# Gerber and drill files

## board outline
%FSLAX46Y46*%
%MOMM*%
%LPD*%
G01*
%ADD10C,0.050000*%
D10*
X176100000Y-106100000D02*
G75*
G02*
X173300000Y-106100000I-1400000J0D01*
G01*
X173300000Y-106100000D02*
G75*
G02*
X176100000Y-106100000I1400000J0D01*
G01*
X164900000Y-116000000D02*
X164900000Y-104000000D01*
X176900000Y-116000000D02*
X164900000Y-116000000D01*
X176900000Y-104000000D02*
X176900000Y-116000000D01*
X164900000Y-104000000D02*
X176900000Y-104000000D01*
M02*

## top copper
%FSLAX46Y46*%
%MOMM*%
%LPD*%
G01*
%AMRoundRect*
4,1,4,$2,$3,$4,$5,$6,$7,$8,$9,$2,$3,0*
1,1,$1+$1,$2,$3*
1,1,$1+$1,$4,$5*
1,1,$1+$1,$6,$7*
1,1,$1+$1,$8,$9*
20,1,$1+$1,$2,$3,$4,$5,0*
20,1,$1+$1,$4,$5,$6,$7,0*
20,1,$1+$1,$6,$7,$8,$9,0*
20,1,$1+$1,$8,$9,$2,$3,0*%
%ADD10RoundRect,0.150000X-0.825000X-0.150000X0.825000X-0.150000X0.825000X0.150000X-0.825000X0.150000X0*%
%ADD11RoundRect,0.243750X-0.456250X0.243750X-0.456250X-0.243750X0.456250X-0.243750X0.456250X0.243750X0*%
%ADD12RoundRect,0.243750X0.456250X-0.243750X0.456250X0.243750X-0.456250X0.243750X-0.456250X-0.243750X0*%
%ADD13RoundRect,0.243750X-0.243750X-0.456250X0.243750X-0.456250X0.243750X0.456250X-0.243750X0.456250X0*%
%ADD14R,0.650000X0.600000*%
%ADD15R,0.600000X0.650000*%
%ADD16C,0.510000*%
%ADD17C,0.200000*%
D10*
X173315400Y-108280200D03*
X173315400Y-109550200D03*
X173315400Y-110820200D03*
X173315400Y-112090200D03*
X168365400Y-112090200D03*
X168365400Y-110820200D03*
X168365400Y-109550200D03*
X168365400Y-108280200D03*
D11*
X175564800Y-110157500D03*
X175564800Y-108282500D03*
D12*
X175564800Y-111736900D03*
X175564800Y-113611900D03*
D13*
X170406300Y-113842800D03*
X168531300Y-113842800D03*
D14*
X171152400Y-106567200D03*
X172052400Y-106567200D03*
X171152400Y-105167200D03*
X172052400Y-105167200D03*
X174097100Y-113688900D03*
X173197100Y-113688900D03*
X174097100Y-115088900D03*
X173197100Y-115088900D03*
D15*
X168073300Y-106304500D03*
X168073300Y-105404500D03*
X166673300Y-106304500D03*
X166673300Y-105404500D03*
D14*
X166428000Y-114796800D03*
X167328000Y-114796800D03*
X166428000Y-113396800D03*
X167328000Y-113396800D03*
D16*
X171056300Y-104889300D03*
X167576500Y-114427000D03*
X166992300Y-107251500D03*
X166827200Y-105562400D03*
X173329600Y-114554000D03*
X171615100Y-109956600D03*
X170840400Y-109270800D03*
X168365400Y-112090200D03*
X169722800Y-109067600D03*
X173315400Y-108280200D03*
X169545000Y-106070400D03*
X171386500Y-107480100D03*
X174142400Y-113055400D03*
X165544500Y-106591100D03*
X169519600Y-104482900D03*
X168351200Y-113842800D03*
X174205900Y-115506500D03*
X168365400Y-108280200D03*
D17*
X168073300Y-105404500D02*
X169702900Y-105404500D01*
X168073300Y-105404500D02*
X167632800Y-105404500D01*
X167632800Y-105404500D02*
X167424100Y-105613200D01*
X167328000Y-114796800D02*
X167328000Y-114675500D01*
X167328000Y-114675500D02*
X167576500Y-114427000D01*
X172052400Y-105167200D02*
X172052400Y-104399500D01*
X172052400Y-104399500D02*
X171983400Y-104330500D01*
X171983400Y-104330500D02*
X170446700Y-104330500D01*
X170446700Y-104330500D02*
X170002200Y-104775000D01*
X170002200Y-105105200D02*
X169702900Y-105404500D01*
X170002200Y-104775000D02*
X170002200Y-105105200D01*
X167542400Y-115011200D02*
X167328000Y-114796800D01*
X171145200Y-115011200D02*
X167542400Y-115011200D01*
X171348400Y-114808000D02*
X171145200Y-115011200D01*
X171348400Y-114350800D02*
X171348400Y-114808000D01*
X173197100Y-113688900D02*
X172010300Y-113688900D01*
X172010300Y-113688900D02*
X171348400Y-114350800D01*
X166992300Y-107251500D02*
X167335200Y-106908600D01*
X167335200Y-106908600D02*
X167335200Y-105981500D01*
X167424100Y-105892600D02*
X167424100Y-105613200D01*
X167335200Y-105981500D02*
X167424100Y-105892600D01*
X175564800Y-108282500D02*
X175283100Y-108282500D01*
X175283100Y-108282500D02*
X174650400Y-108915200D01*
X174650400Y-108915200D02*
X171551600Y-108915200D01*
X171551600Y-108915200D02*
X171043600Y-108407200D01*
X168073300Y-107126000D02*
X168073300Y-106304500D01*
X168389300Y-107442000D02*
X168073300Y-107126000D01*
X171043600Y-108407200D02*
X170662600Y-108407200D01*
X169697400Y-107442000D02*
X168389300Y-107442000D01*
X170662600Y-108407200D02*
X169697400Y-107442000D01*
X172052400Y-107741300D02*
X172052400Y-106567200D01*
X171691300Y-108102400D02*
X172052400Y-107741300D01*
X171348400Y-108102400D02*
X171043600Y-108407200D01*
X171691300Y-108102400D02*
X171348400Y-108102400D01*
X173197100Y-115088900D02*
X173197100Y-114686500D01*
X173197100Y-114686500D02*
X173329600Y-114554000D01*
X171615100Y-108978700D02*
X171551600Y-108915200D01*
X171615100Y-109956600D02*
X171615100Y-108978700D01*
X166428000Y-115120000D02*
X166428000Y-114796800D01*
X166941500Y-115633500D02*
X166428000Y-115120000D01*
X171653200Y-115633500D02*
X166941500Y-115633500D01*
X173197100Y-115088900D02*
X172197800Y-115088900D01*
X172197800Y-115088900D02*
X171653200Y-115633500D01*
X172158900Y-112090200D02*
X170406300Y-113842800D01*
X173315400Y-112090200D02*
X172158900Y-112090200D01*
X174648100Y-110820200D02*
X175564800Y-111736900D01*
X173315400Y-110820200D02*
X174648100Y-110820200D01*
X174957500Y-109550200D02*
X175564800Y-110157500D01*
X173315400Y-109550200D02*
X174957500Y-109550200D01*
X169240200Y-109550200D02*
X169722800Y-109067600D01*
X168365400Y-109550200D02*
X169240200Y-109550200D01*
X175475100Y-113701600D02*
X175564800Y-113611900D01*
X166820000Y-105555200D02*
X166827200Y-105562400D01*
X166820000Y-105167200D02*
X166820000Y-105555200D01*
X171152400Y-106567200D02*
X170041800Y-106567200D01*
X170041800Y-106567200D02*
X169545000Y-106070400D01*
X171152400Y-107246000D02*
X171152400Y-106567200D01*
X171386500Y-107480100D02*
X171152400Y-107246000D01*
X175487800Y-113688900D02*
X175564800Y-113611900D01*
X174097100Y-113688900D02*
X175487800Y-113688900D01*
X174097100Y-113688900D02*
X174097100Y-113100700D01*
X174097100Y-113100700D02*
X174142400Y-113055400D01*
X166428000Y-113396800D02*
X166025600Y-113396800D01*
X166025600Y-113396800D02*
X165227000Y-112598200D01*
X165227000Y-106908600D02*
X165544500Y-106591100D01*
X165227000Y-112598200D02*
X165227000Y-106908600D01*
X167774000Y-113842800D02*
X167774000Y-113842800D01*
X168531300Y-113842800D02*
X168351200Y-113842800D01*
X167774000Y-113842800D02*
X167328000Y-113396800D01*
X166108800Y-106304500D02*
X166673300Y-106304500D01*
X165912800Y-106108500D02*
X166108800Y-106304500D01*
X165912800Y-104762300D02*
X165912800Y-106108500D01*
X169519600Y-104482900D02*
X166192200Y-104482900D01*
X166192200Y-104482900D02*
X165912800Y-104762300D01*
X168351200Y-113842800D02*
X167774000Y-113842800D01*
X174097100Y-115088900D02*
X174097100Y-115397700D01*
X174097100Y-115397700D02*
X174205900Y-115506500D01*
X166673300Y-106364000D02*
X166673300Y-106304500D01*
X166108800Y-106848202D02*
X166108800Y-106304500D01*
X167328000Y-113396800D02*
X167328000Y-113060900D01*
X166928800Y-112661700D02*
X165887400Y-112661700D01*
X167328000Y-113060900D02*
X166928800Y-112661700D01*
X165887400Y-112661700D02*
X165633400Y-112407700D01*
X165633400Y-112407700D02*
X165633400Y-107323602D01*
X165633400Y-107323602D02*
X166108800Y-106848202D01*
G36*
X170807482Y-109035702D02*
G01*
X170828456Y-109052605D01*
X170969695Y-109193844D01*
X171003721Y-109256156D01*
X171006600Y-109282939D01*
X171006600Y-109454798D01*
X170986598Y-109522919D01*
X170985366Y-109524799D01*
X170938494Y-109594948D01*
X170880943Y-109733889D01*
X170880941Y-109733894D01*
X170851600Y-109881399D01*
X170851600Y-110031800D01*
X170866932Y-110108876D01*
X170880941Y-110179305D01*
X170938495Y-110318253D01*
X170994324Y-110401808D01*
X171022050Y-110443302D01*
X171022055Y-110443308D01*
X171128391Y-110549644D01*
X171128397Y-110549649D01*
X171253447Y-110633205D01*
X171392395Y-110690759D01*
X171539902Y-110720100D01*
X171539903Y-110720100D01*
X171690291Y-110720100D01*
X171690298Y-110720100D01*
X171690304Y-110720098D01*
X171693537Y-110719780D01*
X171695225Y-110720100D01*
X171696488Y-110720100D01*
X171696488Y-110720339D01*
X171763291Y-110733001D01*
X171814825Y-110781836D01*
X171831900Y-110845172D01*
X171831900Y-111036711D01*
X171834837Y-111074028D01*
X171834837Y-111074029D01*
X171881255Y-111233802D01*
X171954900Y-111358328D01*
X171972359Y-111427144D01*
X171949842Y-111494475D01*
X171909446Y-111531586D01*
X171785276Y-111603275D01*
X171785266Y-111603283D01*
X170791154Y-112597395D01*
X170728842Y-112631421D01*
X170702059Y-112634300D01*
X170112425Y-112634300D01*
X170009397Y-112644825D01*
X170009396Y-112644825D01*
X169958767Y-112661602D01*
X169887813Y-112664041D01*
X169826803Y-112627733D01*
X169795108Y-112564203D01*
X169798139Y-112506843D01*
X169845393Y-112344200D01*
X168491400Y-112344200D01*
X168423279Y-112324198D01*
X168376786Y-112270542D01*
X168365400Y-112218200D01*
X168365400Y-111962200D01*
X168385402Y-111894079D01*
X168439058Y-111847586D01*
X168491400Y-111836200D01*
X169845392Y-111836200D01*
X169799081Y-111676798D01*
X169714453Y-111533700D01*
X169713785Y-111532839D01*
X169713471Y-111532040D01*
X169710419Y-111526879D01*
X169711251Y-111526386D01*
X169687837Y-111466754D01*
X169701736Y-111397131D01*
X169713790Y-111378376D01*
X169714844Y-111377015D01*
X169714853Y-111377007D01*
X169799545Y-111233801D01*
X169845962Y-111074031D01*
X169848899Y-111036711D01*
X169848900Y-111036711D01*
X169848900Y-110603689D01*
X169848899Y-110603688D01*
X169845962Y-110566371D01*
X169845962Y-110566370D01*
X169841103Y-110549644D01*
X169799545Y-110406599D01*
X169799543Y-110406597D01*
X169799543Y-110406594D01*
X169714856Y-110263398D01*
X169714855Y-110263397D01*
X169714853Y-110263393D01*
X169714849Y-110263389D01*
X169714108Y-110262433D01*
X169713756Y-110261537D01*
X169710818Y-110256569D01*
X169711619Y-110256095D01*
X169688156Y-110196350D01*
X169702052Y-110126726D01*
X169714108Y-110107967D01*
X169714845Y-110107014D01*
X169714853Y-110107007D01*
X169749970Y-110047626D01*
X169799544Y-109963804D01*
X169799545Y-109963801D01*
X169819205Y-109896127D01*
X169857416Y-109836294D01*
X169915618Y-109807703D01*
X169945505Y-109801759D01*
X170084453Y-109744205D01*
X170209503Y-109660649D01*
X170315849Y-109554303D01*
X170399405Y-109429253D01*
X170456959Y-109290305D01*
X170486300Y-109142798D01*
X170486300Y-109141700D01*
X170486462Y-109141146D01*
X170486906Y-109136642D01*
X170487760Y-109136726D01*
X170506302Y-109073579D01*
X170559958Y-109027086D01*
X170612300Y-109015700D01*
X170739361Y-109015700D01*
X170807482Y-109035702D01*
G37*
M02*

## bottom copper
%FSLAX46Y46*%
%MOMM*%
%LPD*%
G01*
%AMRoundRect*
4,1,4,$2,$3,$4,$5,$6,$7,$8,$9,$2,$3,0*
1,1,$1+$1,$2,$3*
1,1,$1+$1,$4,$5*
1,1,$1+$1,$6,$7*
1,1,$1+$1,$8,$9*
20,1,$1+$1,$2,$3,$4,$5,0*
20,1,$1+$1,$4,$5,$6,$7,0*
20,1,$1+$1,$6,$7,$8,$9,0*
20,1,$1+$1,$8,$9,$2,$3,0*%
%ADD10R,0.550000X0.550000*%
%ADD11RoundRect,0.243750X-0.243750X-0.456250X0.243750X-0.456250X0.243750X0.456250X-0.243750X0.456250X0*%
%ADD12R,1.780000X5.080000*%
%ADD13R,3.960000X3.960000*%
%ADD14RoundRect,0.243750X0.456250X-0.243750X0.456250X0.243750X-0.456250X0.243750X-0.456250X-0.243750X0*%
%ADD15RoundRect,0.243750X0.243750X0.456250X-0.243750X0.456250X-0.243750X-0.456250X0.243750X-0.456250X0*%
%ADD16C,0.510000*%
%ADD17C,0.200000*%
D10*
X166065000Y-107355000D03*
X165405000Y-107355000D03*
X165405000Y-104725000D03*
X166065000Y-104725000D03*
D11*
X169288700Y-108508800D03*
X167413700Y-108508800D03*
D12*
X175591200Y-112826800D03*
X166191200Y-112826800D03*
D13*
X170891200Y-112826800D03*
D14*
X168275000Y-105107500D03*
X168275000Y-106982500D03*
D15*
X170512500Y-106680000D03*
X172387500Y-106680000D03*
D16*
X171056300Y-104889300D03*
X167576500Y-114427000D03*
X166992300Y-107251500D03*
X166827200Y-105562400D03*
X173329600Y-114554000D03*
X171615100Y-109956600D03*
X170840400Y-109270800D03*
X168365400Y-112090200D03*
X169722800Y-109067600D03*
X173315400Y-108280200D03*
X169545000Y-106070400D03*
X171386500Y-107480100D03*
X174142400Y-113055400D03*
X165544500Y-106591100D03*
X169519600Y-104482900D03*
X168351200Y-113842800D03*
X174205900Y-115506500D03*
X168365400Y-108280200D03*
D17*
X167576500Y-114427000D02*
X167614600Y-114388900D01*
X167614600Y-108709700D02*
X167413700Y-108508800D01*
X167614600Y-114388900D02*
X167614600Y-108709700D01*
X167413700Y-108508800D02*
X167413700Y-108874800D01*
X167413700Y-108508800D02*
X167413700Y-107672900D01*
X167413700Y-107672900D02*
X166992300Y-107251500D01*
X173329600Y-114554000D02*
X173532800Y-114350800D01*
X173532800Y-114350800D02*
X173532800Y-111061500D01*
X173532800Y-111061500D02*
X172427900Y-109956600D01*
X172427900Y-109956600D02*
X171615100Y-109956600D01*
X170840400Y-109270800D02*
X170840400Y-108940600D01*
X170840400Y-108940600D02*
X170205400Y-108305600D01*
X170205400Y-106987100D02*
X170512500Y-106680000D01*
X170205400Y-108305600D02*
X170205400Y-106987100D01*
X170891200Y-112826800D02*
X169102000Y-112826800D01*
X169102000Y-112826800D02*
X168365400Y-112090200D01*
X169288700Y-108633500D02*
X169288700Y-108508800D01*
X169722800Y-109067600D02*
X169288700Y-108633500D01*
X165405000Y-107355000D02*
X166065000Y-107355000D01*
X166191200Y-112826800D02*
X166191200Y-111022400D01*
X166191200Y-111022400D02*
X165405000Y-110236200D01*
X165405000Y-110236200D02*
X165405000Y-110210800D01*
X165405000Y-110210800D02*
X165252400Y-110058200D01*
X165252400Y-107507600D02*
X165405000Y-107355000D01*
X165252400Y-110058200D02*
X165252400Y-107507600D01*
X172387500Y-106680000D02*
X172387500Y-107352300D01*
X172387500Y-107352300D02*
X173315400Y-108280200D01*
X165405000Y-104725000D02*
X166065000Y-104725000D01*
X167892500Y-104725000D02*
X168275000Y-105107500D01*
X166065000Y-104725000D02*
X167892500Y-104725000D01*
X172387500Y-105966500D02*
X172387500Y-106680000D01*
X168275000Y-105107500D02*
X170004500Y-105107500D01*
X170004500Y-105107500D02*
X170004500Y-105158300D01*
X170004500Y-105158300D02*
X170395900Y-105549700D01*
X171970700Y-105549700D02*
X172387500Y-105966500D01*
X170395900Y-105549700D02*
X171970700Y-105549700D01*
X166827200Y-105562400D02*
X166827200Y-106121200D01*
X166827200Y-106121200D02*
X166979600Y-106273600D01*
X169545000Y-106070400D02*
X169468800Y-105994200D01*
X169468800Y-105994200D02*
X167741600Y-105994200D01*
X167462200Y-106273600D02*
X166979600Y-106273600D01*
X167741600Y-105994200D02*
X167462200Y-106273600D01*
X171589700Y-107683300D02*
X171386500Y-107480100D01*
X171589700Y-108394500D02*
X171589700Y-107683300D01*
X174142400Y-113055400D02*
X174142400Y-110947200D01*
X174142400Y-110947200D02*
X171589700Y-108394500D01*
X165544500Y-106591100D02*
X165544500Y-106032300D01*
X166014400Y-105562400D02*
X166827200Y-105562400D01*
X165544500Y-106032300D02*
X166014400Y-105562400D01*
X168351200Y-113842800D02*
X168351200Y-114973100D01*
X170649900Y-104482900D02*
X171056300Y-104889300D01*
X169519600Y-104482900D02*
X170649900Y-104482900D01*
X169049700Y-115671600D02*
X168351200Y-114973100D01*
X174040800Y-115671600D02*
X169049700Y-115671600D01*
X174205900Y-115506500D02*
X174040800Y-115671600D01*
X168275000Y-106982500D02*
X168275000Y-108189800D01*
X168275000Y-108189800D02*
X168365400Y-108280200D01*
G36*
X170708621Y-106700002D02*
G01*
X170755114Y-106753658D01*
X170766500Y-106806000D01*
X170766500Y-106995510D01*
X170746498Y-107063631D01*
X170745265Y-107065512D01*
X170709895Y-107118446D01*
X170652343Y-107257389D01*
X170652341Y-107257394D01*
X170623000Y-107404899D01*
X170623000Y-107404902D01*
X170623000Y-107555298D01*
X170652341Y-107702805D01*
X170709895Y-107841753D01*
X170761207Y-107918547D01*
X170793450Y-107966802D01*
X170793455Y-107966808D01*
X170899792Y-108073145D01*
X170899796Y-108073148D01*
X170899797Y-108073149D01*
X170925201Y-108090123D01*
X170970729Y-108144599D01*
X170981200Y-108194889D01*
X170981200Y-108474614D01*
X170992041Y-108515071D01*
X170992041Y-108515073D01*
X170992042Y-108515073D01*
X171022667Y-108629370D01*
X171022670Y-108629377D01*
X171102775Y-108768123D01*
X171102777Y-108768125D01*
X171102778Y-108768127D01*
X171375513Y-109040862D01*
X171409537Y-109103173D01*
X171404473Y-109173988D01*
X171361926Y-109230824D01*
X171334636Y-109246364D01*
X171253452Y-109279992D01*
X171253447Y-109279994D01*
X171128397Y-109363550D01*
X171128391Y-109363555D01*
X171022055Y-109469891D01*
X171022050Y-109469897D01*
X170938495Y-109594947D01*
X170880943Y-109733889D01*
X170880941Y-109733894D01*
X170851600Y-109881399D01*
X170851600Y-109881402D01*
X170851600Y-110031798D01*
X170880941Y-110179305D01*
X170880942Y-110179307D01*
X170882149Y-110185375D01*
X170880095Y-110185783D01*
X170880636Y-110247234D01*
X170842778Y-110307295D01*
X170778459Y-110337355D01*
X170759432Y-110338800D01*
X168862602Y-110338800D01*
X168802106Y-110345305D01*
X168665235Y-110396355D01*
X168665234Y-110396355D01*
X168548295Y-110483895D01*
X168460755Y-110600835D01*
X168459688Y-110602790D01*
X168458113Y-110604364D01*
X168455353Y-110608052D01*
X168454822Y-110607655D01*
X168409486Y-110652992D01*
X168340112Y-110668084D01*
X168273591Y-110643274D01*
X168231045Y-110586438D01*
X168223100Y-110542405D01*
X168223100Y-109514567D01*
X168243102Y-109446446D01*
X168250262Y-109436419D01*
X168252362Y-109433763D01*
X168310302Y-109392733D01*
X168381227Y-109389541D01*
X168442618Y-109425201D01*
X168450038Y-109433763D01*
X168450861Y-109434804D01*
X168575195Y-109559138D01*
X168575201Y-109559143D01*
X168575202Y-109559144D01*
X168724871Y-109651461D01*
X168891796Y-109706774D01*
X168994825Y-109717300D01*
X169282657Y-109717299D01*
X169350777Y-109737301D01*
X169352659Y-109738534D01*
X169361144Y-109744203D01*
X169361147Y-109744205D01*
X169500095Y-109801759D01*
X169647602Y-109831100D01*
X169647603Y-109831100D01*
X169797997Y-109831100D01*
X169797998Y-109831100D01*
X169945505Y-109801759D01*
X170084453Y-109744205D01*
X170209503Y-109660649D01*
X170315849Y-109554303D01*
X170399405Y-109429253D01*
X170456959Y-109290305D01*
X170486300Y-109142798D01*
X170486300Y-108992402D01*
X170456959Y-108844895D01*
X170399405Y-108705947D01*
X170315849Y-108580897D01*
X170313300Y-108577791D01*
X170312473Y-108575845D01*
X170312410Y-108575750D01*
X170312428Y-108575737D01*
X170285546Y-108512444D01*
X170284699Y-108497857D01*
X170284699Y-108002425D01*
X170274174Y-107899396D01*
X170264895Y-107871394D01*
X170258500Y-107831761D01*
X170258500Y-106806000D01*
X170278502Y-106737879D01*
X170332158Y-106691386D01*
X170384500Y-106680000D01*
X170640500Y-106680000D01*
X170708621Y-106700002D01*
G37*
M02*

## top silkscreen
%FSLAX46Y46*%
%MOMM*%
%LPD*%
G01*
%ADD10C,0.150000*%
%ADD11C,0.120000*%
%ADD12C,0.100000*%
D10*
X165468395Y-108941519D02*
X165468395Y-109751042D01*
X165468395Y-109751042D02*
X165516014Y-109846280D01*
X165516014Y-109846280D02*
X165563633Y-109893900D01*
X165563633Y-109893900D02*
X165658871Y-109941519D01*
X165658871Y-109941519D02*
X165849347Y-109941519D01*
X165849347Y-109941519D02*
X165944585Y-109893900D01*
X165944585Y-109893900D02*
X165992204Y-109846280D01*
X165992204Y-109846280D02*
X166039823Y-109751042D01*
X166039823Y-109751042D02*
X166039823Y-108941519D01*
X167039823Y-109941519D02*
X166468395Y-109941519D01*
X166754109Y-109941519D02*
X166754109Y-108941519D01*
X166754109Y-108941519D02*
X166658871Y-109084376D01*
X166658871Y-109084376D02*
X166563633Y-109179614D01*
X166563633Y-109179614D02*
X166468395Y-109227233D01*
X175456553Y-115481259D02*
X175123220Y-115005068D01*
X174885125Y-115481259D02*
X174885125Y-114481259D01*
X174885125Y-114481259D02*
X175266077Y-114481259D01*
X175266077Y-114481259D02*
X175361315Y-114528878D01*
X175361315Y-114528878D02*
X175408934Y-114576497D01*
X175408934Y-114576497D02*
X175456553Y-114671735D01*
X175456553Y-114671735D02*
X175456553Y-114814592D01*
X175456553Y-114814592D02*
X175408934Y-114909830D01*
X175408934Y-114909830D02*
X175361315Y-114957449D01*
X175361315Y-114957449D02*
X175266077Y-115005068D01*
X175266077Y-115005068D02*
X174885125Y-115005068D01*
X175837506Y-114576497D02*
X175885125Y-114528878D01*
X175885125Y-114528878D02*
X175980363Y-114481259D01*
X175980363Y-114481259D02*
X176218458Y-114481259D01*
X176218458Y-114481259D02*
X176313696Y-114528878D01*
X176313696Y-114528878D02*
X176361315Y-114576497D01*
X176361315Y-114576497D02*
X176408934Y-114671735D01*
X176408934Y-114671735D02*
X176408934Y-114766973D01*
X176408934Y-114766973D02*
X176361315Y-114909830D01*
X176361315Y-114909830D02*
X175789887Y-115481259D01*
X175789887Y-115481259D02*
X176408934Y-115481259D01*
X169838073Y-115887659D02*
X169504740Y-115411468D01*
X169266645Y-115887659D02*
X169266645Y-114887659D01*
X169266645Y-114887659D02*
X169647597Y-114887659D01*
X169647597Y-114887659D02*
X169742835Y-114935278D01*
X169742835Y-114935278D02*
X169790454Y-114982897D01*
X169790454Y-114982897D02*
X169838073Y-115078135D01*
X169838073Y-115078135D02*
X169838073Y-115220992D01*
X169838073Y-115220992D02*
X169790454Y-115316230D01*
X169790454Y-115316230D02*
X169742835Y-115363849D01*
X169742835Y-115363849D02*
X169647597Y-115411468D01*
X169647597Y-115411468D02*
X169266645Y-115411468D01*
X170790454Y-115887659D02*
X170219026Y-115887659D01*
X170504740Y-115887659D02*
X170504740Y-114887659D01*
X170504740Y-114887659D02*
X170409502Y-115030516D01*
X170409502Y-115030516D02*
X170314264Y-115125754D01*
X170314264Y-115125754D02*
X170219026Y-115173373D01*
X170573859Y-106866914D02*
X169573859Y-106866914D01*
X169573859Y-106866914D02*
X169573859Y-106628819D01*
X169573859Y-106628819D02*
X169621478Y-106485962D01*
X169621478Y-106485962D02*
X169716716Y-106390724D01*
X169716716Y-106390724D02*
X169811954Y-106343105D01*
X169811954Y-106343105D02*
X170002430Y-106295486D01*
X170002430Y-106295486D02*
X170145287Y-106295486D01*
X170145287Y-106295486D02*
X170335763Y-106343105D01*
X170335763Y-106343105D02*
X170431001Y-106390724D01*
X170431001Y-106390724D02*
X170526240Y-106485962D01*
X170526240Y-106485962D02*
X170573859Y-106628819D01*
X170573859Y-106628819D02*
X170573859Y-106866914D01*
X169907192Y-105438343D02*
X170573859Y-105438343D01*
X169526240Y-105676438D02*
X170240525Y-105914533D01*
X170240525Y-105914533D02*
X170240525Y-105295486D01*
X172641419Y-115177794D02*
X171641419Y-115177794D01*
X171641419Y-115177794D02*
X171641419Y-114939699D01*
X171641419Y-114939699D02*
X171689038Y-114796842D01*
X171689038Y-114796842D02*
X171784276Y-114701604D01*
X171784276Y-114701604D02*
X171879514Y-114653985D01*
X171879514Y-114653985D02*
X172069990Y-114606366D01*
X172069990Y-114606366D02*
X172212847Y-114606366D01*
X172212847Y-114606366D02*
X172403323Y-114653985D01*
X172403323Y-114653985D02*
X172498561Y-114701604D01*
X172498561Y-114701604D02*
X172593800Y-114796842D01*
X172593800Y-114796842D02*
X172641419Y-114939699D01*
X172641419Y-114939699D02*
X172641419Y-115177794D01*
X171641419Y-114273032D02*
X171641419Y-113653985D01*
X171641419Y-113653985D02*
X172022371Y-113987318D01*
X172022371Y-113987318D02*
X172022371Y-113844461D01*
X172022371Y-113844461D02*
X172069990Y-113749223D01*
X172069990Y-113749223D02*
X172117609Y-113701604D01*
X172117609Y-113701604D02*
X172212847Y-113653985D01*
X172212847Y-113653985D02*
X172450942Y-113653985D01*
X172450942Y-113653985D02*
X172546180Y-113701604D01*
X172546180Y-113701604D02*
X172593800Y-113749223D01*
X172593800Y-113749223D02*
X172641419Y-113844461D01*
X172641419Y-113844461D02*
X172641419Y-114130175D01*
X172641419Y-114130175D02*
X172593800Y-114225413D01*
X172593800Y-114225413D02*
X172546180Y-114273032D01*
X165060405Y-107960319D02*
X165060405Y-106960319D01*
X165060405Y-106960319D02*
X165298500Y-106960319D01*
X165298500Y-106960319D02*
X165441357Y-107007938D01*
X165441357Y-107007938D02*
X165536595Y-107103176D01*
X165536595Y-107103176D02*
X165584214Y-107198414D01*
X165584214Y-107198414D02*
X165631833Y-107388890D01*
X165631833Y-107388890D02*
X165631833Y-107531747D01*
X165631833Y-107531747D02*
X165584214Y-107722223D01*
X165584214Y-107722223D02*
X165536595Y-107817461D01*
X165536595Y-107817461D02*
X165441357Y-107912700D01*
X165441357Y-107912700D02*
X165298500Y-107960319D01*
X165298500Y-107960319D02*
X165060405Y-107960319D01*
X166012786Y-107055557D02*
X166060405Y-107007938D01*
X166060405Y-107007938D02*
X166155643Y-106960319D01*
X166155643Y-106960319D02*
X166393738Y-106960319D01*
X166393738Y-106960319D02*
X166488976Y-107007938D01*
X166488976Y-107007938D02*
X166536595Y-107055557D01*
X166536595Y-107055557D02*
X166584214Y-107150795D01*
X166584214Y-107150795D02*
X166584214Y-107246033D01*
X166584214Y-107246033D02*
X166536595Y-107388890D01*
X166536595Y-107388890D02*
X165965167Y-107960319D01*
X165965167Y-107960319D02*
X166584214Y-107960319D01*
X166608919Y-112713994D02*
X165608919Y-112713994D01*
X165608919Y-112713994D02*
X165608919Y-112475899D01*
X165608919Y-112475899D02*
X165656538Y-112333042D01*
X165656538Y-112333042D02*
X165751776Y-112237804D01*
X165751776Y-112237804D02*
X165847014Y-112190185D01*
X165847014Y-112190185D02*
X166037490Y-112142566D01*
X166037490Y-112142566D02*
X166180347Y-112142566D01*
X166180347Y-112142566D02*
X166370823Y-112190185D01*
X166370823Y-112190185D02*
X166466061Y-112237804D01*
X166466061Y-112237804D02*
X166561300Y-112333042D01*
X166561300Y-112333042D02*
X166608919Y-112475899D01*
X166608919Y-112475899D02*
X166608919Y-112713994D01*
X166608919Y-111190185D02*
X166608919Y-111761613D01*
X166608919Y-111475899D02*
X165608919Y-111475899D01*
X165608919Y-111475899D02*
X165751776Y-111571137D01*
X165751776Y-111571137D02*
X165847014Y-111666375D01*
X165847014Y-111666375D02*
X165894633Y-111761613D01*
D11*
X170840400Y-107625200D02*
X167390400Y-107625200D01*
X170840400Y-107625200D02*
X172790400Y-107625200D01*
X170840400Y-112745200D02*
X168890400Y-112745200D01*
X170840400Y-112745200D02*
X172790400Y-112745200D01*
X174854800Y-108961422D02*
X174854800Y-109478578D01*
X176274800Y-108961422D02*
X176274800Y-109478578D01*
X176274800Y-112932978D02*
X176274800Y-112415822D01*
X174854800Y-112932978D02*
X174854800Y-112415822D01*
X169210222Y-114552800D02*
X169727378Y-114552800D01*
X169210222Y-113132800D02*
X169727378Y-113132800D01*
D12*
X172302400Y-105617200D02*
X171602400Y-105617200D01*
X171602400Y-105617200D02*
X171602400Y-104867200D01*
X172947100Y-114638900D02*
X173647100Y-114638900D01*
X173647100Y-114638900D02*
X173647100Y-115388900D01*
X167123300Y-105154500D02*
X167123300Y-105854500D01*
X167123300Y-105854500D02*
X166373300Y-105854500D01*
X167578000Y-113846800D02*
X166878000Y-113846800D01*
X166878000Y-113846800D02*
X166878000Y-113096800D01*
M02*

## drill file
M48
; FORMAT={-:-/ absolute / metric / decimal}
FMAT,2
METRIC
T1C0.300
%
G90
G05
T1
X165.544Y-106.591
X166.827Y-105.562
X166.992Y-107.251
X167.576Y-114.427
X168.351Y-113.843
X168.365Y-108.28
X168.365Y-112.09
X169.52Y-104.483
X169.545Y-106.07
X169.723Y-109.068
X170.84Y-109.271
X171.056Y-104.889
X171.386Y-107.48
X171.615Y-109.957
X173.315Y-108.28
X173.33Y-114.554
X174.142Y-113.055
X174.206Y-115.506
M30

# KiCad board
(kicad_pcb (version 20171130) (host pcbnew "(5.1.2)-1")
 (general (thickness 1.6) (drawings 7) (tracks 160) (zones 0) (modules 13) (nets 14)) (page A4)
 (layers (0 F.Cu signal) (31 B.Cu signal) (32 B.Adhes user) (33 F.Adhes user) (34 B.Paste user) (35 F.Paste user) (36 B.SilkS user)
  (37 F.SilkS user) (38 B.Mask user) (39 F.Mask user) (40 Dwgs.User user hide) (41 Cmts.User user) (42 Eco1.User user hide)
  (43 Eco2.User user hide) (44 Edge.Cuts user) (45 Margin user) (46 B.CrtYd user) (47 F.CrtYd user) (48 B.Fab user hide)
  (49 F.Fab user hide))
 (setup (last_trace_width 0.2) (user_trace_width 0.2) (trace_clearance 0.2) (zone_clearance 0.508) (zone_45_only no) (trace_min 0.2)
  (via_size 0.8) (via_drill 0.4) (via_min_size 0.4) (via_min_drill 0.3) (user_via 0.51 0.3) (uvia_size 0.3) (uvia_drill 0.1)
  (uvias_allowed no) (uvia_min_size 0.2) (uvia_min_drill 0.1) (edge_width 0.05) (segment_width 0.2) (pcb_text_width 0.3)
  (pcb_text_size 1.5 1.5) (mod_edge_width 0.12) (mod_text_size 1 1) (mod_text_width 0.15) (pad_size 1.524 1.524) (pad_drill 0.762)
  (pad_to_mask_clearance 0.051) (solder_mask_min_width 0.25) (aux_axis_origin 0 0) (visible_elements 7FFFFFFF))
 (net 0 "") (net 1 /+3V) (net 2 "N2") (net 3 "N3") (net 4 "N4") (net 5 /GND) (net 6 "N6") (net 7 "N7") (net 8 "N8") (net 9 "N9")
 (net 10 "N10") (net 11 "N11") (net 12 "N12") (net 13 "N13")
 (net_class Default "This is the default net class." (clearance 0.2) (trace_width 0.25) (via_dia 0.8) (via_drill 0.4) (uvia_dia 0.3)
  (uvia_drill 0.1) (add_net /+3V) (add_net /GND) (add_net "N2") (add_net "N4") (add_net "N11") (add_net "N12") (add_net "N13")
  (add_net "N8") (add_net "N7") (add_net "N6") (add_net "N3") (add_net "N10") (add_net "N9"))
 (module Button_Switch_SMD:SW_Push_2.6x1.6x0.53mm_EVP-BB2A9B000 (layer B.Cu) (at 165.735 106.045 90)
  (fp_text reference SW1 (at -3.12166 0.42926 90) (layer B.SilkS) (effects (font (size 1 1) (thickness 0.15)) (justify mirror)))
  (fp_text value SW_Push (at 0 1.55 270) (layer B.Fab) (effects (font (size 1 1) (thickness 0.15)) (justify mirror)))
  (pad 1 smd rect (at -1.31 0.33 90) (size 0.55 0.55) (layers B.Cu B.Paste B.Mask) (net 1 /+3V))
  (pad 1 smd rect (at -1.31 -0.33 90) (size 0.55 0.55) (layers B.Cu B.Paste B.Mask) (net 1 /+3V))
  (pad 2 smd rect (at 1.32 -0.33 90) (size 0.55 0.55) (layers B.Cu B.Paste B.Mask) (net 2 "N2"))
  (pad 2 smd rect (at 1.32 0.33 90) (size 0.55 0.55) (layers B.Cu B.Paste B.Mask) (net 2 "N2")))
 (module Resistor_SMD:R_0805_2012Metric (layer B.Cu) (at 168.3512 108.5088)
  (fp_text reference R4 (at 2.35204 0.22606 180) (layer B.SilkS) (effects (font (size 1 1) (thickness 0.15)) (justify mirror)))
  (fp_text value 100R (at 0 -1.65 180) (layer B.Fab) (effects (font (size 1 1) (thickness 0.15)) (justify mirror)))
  (pad 2 smd roundrect (at 0.9375 0) (size 0.975 1.4) (layers B.Cu B.Paste B.Mask) (roundrect_rratio 0.25) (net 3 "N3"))
  (pad 1 smd roundrect (at -0.9375 0) (size 0.975 1.4) (layers B.Cu B.Paste B.Mask) (roundrect_rratio 0.25) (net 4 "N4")))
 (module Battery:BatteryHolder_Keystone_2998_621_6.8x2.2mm (layer B.Cu) (at 170.8912 112.8268)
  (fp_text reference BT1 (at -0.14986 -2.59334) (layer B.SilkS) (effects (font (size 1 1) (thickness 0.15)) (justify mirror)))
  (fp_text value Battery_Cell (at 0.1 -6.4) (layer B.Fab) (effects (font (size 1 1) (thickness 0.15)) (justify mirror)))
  (pad 1 smd rect (at 4.7 0) (size 1.78 5.08) (layers B.Cu B.Paste B.Mask) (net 1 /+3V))
  (pad 1 smd rect (at -4.7 0) (size 1.78 5.08) (layers B.Cu B.Paste B.Mask) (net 1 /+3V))
  (pad 2 smd rect (at 0 0) (size 3.96 3.96) (layers B.Cu B.Paste B.Mask) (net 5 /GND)))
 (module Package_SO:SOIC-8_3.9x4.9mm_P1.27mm (layer F.Cu) (at 170.8404 110.1852)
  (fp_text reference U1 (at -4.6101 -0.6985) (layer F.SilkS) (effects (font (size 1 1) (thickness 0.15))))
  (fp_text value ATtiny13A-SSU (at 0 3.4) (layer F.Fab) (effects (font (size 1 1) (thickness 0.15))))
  (fp_line (start 0 -2.56) (end -3.45 -2.56) (layer F.SilkS) (width 0.12))
  (fp_line (start 0 -2.56) (end 1.95 -2.56) (layer F.SilkS) (width 0.12))
  (fp_line (start 0 2.56) (end -1.95 2.56) (layer F.SilkS) (width 0.12))
  (fp_line (start 0 2.56) (end 1.95 2.56) (layer F.SilkS) (width 0.12))
  (pad 8 smd roundrect (at 2.475 -1.905) (size 1.95 0.6) (layers F.Cu F.Paste F.Mask) (roundrect_rratio 0.25) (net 2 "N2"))
  (pad 7 smd roundrect (at 2.475 -0.635) (size 1.95 0.6) (layers F.Cu F.Paste F.Mask) (roundrect_rratio 0.25) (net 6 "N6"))
  (pad 6 smd roundrect (at 2.475 0.635) (size 1.95 0.6) (layers F.Cu F.Paste F.Mask) (roundrect_rratio 0.25) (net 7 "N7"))
  (pad 5 smd roundrect (at 2.475 1.905) (size 1.95 0.6) (layers F.Cu F.Paste F.Mask) (roundrect_rratio 0.25) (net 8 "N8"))
  (pad 4 smd roundrect (at -2.475 1.905) (size 1.95 0.6) (layers F.Cu F.Paste F.Mask) (roundrect_rratio 0.25) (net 5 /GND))
  (pad 3 smd roundrect (at -2.475 0.635) (size 1.95 0.6) (layers F.Cu F.Paste F.Mask) (roundrect_rratio 0.25) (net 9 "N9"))
  (pad 2 smd roundrect (at -2.475 -0.635) (size 1.95 0.6) (layers F.Cu F.Paste F.Mask) (roundrect_rratio 0.25) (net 3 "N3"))
  (pad 1 smd roundrect (at -2.475 -1.905) (size 1.95 0.6) (layers F.Cu F.Paste F.Mask) (roundrect_rratio 0.25) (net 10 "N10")))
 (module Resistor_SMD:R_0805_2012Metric (layer B.Cu) (at 168.275 106.045 90)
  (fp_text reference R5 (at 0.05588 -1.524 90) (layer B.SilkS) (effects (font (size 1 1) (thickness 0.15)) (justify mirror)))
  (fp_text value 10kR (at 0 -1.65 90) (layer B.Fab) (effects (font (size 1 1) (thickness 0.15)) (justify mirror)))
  (pad 2 smd roundrect (at 0.9375 0 90) (size 0.975 1.4) (layers B.Cu B.Paste B.Mask) (roundrect_rratio 0.25) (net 2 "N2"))
  (pad 1 smd roundrect (at -0.9375 0 90) (size 0.975 1.4) (layers B.Cu B.Paste B.Mask) (roundrect_rratio 0.25) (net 10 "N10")))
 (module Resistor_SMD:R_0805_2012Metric (layer F.Cu) (at 175.5648 109.22 270)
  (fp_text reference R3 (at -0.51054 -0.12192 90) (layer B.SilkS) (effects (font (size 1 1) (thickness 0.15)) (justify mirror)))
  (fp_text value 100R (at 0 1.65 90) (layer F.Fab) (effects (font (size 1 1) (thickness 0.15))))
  (fp_line (start -0.258578 0.71) (end 0.258578 0.71) (layer F.SilkS) (width 0.12))
  (fp_line (start -0.258578 -0.71) (end 0.258578 -0.71) (layer F.SilkS) (width 0.12))
  (pad 2 smd roundrect (at 0.9375 0 270) (size 0.975 1.4) (layers F.Cu F.Paste F.Mask) (roundrect_rratio 0.25) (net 6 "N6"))
  (pad 1 smd roundrect (at -0.9375 0 270) (size 0.975 1.4) (layers F.Cu F.Paste F.Mask) (roundrect_rratio 0.25) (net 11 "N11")))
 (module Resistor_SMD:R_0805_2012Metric (layer F.Cu) (at 175.5648 112.6744 90)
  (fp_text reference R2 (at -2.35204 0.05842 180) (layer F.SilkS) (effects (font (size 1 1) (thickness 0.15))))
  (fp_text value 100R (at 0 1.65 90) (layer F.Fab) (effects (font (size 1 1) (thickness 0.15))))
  (fp_line (start -0.258578 0.71) (end 0.258578 0.71) (layer F.SilkS) (width 0.12))
  (fp_line (start -0.258578 -0.71) (end 0.258578 -0.71) (layer F.SilkS) (width 0.12))
  (pad 2 smd roundrect (at 0.9375 0 90) (size 0.975 1.4) (layers F.Cu F.Paste F.Mask) (roundrect_rratio 0.25) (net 7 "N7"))
  (pad 1 smd roundrect (at -0.9375 0 90) (size 0.975 1.4) (layers F.Cu F.Paste F.Mask) (roundrect_rratio 0.25) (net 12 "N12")))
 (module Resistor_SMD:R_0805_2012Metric (layer F.Cu) (at 169.4688 113.8428)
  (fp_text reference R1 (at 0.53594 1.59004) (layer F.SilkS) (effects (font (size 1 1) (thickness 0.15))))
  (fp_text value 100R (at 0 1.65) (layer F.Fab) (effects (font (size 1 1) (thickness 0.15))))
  (fp_line (start -0.258578 0.71) (end 0.258578 0.71) (layer F.SilkS) (width 0.12))
  (fp_line (start -0.258578 -0.71) (end 0.258578 -0.71) (layer F.SilkS) (width 0.12))
  (pad 2 smd roundrect (at 0.9375 0) (size 0.975 1.4) (layers F.Cu F.Paste F.Mask) (roundrect_rratio 0.25) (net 8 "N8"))
  (pad 1 smd roundrect (at -0.9375 0) (size 0.975 1.4) (layers F.Cu F.Paste F.Mask) (roundrect_rratio 0.25) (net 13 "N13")))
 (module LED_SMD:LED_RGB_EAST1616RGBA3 (layer F.Cu) (at 171.6024 105.8672 90)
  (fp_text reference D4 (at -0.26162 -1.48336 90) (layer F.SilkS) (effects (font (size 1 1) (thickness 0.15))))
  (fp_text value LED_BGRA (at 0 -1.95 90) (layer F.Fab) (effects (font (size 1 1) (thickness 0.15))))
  (fp_line (start 0.25 0.7) (end 0.25 0) (layer F.SilkS) (width 0.1))
  (fp_line (start 0.25 0) (end 1 0) (layer F.SilkS) (width 0.1))
  (pad 2 smd rect (at -0.7 -0.45 90) (size 0.6 0.65) (layers F.Cu F.Paste F.Mask) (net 12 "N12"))
  (pad 1 smd rect (at -0.7 0.45 90) (size 0.6 0.65) (layers F.Cu F.Paste F.Mask) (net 11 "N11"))
  (pad 3 smd rect (at 0.7 -0.45 90) (size 0.6 0.65) (layers F.Cu F.Paste F.Mask) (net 13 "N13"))
  (pad 4 smd rect (at 0.7 0.45 90) (size 0.6 0.65) (layers F.Cu F.Paste F.Mask) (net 4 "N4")))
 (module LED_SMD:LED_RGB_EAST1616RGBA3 (layer F.Cu) (at 173.6471 114.3889 270)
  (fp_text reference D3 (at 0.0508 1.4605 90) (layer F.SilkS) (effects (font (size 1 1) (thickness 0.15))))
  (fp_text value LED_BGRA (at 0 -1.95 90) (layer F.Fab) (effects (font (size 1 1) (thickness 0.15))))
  (fp_line (start 0.25 0.7) (end 0.25 0) (layer F.SilkS) (width 0.1))
  (fp_line (start 0.25 0) (end 1 0) (layer F.SilkS) (width 0.1))
  (pad 2 smd rect (at -0.7 -0.45 270) (size 0.6 0.65) (layers F.Cu F.Paste F.Mask) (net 12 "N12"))
  (pad 1 smd rect (at -0.7 0.45 270) (size 0.6 0.65) (layers F.Cu F.Paste F.Mask) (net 4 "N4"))
  (pad 3 smd rect (at 0.7 -0.45 270) (size 0.6 0.65) (layers F.Cu F.Paste F.Mask) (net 13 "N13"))
  (pad 4 smd rect (at 0.7 0.45 270) (size 0.6 0.65) (layers F.Cu F.Paste F.Mask) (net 11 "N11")))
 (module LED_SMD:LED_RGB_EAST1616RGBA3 (layer F.Cu) (at 167.3733 105.8545 180)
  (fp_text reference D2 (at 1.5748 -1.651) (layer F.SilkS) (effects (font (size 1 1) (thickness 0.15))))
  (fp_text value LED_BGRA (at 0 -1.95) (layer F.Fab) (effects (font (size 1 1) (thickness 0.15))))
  (fp_line (start 0.25 0.7) (end 0.25 0) (layer F.SilkS) (width 0.1))
  (fp_line (start 0.25 0) (end 1 0) (layer F.SilkS) (width 0.1))
  (pad 2 smd rect (at -0.7 -0.45 180) (size 0.6 0.65) (layers F.Cu F.Paste F.Mask) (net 11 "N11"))
  (pad 1 smd rect (at -0.7 0.45 180) (size 0.6 0.65) (layers F.Cu F.Paste F.Mask) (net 4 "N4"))
  (pad 3 smd rect (at 0.7 -0.45 180) (size 0.6 0.65) (layers F.Cu F.Paste F.Mask) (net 13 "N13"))
  (pad 4 smd rect (at 0.7 0.45 180) (size 0.6 0.65) (layers F.Cu F.Paste F.Mask) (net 12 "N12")))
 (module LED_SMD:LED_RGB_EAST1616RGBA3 (layer F.Cu) (at 166.878 114.0968 90)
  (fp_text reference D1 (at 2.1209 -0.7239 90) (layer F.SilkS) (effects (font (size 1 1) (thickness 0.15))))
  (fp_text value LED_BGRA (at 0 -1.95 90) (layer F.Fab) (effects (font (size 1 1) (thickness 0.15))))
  (fp_line (start 0.25 0.7) (end 0.25 0) (layer F.SilkS) (width 0.1))
  (fp_line (start 0.25 0) (end 1 0) (layer F.SilkS) (width 0.1))
  (pad 2 smd rect (at -0.7 -0.45 90) (size 0.6 0.65) (layers F.Cu F.Paste F.Mask) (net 11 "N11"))
  (pad 1 smd rect (at -0.7 0.45 90) (size 0.6 0.65) (layers F.Cu F.Paste F.Mask) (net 4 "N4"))
  (pad 3 smd rect (at 0.7 -0.45 90) (size 0.6 0.65) (layers F.Cu F.Paste F.Mask) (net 12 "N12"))
  (pad 4 smd rect (at 0.7 0.45 90) (size 0.6 0.65) (layers F.Cu F.Paste F.Mask) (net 13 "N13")))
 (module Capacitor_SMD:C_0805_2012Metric (layer B.Cu) (at 171.45 106.68 180)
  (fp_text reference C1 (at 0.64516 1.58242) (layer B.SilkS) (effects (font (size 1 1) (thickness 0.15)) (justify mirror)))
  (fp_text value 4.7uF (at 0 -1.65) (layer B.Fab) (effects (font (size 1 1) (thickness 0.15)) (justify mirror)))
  (pad 2 smd roundrect (at 0.9375 0 180) (size 0.975 1.4) (layers B.Cu B.Paste B.Mask) (roundrect_rratio 0.25) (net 5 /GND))
  (pad 1 smd roundrect (at -0.9375 0 180) (size 0.975 1.4) (layers B.Cu B.Paste B.Mask) (roundrect_rratio 0.25) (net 2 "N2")))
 (gr_circle (center 174.7 106.1) (end 176.1 106.1) (layer Edge.Cuts) (width 0.05))
 (gr_line (start 164.9 116) (end 164.9 104) (layer Edge.Cuts) (width 0.05))
 (gr_line (start 176.9 116) (end 164.9 116) (layer Edge.Cuts) (width 0.05))
 (gr_line (start 176.9 104) (end 176.9 116) (layer Edge.Cuts) (width 0.05))
 (gr_line (start 164.9 104) (end 176.9 104) (layer Edge.Cuts) (width 0.05))
 (via (at 171.0563 104.8893) (size 0.51) (drill 0.3) (layers F.Cu B.Cu) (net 13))
 (segment (start 168.0733 105.4045) (end 169.7029 105.4045) (width 0.2) (layer F.Cu) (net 4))
 (segment (start 168.0733 105.4045) (end 167.6328 105.4045) (width 0.2) (layer F.Cu) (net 4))
 (segment (start 167.6328 105.4045) (end 167.4241 105.6132) (width 0.2) (layer F.Cu) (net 4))
 (via (at 167.5765 114.427) (size 0.51) (drill 0.3) (layers F.Cu B.Cu) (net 4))
 (segment (start 167.328 114.7968) (end 167.328 114.6755) (width 0.2) (layer F.Cu) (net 4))
 (segment (start 167.328 114.6755) (end 167.5765 114.427) (width 0.2) (layer F.Cu) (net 4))
 (segment (start 167.5765 114.427) (end 167.6146 114.3889) (width 0.2) (layer B.Cu) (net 4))
 (segment (start 167.6146 108.7097) (end 167.4137 108.5088) (width 0.2) (layer B.Cu) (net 4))
 (segment (start 167.6146 114.3889) (end 167.6146 108.7097) (width 0.2) (layer B.Cu) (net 4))
 (segment (start 172.0524 105.1672) (end 172.0524 104.3995) (width 0.2) (layer F.Cu) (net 4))
 (segment (start 172.0524 104.3995) (end 171.9834 104.3305) (width 0.2) (layer F.Cu) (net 4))
 (segment (start 171.9834 104.3305) (end 170.4467 104.3305) (width 0.2) (layer F.Cu) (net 4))
 (segment (start 170.4467 104.3305) (end 170.0022 104.775) (width 0.2) (layer F.Cu) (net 4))
 (segment (start 170.0022 105.1052) (end 169.7029 105.4045) (width 0.2) (layer F.Cu) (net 4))
 (segment (start 170.0022 104.775) (end 170.0022 105.1052) (width 0.2) (layer F.Cu) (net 4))
 (segment (start 167.5424 115.0112) (end 167.328 114.7968) (width 0.2) (layer F.Cu) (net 4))
 (segment (start 171.1452 115.0112) (end 167.5424 115.0112) (width 0.2) (layer F.Cu) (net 4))
 (segment (start 171.3484 114.808) (end 171.1452 115.0112) (width 0.2) (layer F.Cu) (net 4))
 (segment (start 171.3484 114.3508) (end 171.3484 114.808) (width 0.2) (layer F.Cu) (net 4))
 (segment (start 173.1971 113.6889) (end 172.0103 113.6889) (width 0.2) (layer F.Cu) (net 4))
 (segment (start 172.0103 113.6889) (end 171.3484 114.3508) (width 0.2) (layer F.Cu) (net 4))
 (segment (start 167.4137 108.5088) (end 167.4137 108.8748) (width 0.2) (layer B.Cu) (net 4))
 (via (at 166.9923 107.2515) (size 0.51) (drill 0.3) (layers F.Cu B.Cu) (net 4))
 (segment (start 167.4137 108.5088) (end 167.4137 107.6729) (width 0.2) (layer B.Cu) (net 4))
 (segment (start 167.4137 107.6729) (end 166.9923 107.2515) (width 0.2) (layer B.Cu) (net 4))
 (segment (start 166.9923 107.2515) (end 167.3352 106.9086) (width 0.2) (layer F.Cu) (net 4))
 (segment (start 167.3352 106.9086) (end 167.3352 105.9815) (width 0.2) (layer F.Cu) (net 4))
 (segment (start 167.4241 105.8926) (end 167.4241 105.6132) (width 0.2) (layer F.Cu) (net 4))
 (segment (start 167.3352 105.9815) (end 167.4241 105.8926) (width 0.2) (layer F.Cu) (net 4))
 (via (at 166.8272 105.5624) (size 0.51) (drill 0.3) (layers F.Cu B.Cu) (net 12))
 (segment (start 175.5648 108.2825) (end 175.2831 108.2825) (width 0.2) (layer F.Cu) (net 11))
 (segment (start 175.2831 108.2825) (end 174.6504 108.9152) (width 0.2) (layer F.Cu) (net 11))
 (segment (start 174.6504 108.9152) (end 171.5516 108.9152) (width 0.2) (layer F.Cu) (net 11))
 (segment (start 171.5516 108.9152) (end 171.0436 108.4072) (width 0.2) (layer F.Cu) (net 11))
 (segment (start 168.0733 107.126) (end 168.0733 106.3045) (width 0.2) (layer F.Cu) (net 11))
 (segment (start 168.3893 107.442) (end 168.0733 107.126) (width 0.2) (layer F.Cu) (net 11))
 (segment (start 171.0436 108.4072) (end 170.6626 108.4072) (width 0.2) (layer F.Cu) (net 11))
 (segment (start 169.6974 107.442) (end 168.3893 107.442) (width 0.2) (layer F.Cu) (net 11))
 (segment (start 170.6626 108.4072) (end 169.6974 107.442) (width 0.2) (layer F.Cu) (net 11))
 (segment (start 172.0524 107.7413) (end 172.0524 106.5672) (width 0.2) (layer F.Cu) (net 11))
 (segment (start 171.6913 108.1024) (end 172.0524 107.7413) (width 0.2) (layer F.Cu) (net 11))
 (segment (start 171.3484 108.1024) (end 171.0436 108.4072) (width 0.2) (layer F.Cu) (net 11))
 (segment (start 171.6913 108.1024) (end 171.3484 108.1024) (width 0.2) (layer F.Cu) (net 11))
 (via (at 173.3296 114.554) (size 0.51) (drill 0.3) (layers F.Cu B.Cu) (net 11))
 (segment (start 173.1971 115.0889) (end 173.1971 114.6865) (width 0.2) (layer F.Cu) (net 11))
 (segment (start 173.1971 114.6865) (end 173.3296 114.554) (width 0.2) (layer F.Cu) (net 11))
 (segment (start 173.3296 114.554) (end 173.5328 114.3508) (width 0.2) (layer B.Cu) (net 11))
 (segment (start 173.5328 114.3508) (end 173.5328 111.0615) (width 0.2) (layer B.Cu) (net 11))
 (via (at 171.6151 109.9566) (size 0.51) (drill 0.3) (layers F.Cu B.Cu) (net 11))
 (segment (start 173.5328 111.0615) (end 172.4279 109.9566) (width 0.2) (layer B.Cu) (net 11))
 (segment (start 172.4279 109.9566) (end 171.6151 109.9566) (width 0.2) (layer B.Cu) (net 11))
 (segment (start 171.6151 108.9787) (end 171.5516 108.9152) (width 0.2) (layer F.Cu) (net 11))
 (segment (start 171.6151 109.9566) (end 171.6151 108.9787) (width 0.2) (layer F.Cu) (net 11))
 (segment (start 166.428 115.12) (end 166.428 114.7968) (width 0.2) (layer F.Cu) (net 11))
 (segment (start 166.9415 115.6335) (end 166.428 115.12) (width 0.2) (layer F.Cu) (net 11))
 (segment (start 171.6532 115.6335) (end 166.9415 115.6335) (width 0.2) (layer F.Cu) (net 11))
 (segment (start 173.1971 115.0889) (end 172.1978 115.0889) (width 0.2) (layer F.Cu) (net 11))
 (segment (start 172.1978 115.0889) (end 171.6532 115.6335) (width 0.2) (layer F.Cu) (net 11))
 (via (at 170.8404 109.2708) (size 0.51) (drill 0.3) (layers F.Cu B.Cu) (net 5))
 (segment (start 170.8404 109.2708) (end 170.8404 108.9406) (width 0.2) (layer B.Cu) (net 5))
 (segment (start 170.8404 108.9406) (end 170.2054 108.3056) (width 0.2) (layer B.Cu) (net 5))
 (segment (start 170.2054 106.9871) (end 170.5125 106.68) (width 0.2) (layer B.Cu) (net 5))
 (segment (start 170.2054 108.3056) (end 170.2054 106.9871) (width 0.2) (layer B.Cu) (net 5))
 (via (at 168.3654 112.0902) (size 0.51) (drill 0.3) (layers F.Cu B.Cu) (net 5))
 (segment (start 170.8912 112.8268) (end 169.102 112.8268) (width 0.2) (layer B.Cu) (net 5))
 (segment (start 169.102 112.8268) (end 168.3654 112.0902) (width 0.2) (layer B.Cu) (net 5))
 (segment (start 172.1589 112.0902) (end 170.4063 113.8428) (width 0.2) (layer F.Cu) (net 8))
 (segment (start 173.3154 112.0902) (end 172.1589 112.0902) (width 0.2) (layer F.Cu) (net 8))
 (segment (start 174.6481 110.8202) (end 175.5648 111.7369) (width 0.2) (layer F.Cu) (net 7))
 (segment (start 173.3154 110.8202) (end 174.6481 110.8202) (width 0.2) (layer F.Cu) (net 7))
 (segment (start 174.9575 109.5502) (end 175.5648 110.1575) (width 0.2) (layer F.Cu) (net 6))
 (segment (start 173.3154 109.5502) (end 174.9575 109.5502) (width 0.2) (layer F.Cu) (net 6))
 (via (at 169.7228 109.0676) (size 0.51) (drill 0.3) (layers F.Cu B.Cu) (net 3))
 (segment (start 169.2402 109.5502) (end 169.7228 109.0676) (width 0.2) (layer F.Cu) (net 3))
 (segment (start 169.2887 108.6335) (end 169.2887 108.5088) (width 0.2) (layer B.Cu) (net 3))
 (segment (start 169.7228 109.0676) (end 169.2887 108.6335) (width 0.2) (layer B.Cu) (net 3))
 (segment (start 168.3654 109.5502) (end 169.2402 109.5502) (width 0.2) (layer F.Cu) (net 3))
 (segment (start 165.405 107.355) (end 166.065 107.355) (width 0.2) (layer B.Cu) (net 1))
 (segment (start 166.1912 112.8268) (end 166.1912 111.0224) (width 0.2) (layer B.Cu) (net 1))
 (segment (start 166.1912 111.0224) (end 165.405 110.2362) (width 0.2) (layer B.Cu) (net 1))
 (segment (start 165.405 110.2362) (end 165.405 110.2108) (width 0.2) (layer B.Cu) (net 1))
 (segment (start 165.405 110.2108) (end 165.2524 110.0582) (width 0.2) (layer B.Cu) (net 1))
 (segment (start 165.2524 107.5076) (end 165.405 107.355) (width 0.2) (layer B.Cu) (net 1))
 (segment (start 165.2524 110.0582) (end 165.2524 107.5076) (width 0.2) (layer B.Cu) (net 1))
 (via (at 173.3154 108.2802) (size 0.51) (drill 0.3) (layers F.Cu B.Cu) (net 2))
 (segment (start 172.3875 106.68) (end 172.3875 107.3523) (width 0.2) (layer B.Cu) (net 2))
 (segment (start 172.3875 107.3523) (end 173.3154 108.2802) (width 0.2) (layer B.Cu) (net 2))
 (segment (start 165.405 104.725) (end 166.065 104.725) (width 0.2) (layer B.Cu) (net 2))
 (segment (start 167.8925 104.725) (end 168.275 105.1075) (width 0.2) (layer B.Cu) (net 2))
 (segment (start 166.065 104.725) (end 167.8925 104.725) (width 0.2) (layer B.Cu) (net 2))
 (segment (start 172.3875 105.9665) (end 172.3875 106.68) (width 0.2) (layer B.Cu) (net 2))
 (segment (start 168.275 105.1075) (end 170.0045 105.1075) (width 0.2) (layer B.Cu) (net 2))
 (segment (start 170.0045 105.1075) (end 170.0045 105.1583) (width 0.2) (layer B.Cu) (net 2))
 (segment (start 170.0045 105.1583) (end 170.3959 105.5497) (width 0.2) (layer B.Cu) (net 2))
 (segment (start 171.9707 105.5497) (end 172.3875 105.9665) (width 0.2) (layer B.Cu) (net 2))
 (segment (start 170.3959 105.5497) (end 171.9707 105.5497) (width 0.2) (layer B.Cu) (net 2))
 (segment (start 175.4751 113.7016) (end 175.5648 113.6119) (width 0.2) (layer F.Cu) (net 12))
 (segment (start 166.82 105.5552) (end 166.8272 105.5624) (width 0.2) (layer F.Cu) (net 12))
 (segment (start 166.82 105.1672) (end 166.82 105.5552) (width 0.2) (layer F.Cu) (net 12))
 (segment (start 166.8272 105.5624) (end 166.8272 106.1212) (width 0.2) (layer B.Cu) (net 12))
 (segment (start 166.8272 106.1212) (end 166.9796 106.2736) (width 0.2) (layer B.Cu) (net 12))
 (via (at 169.545 106.0704) (size 0.51) (drill 0.3) (layers F.Cu B.Cu) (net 12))
 (segment (start 171.1524 106.5672) (end 170.0418 106.5672) (width 0.2) (layer F.Cu) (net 12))
 (segment (start 170.0418 106.5672) (end 169.545 106.0704) (width 0.2) (layer F.Cu) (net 12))
 (segment (start 169.545 106.0704) (end 169.4688 105.9942) (width 0.2) (layer B.Cu) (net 12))
 (segment (start 169.4688 105.9942) (end 167.7416 105.9942) (width 0.2) (layer B.Cu) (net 12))
 (segment (start 167.4622 106.2736) (end 166.9796 106.2736) (width 0.2) (layer B.Cu) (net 12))
 (segment (start 167.7416 105.9942) (end 167.4622 106.2736) (width 0.2) (layer B.Cu) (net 12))
 (via (at 171.3865 107.4801) (size 0.51) (drill 0.3) (layers F.Cu B.Cu) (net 12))
 (segment (start 171.1524 107.246) (end 171.1524 106.5672) (width 0.2) (layer F.Cu) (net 12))
 (segment (start 171.3865 107.4801) (end 171.1524 107.246) (width 0.2) (layer F.Cu) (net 12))
 (segment (start 175.4878 113.6889) (end 175.5648 113.6119) (width 0.2) (layer F.Cu) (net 12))
 (segment (start 174.0971 113.6889) (end 175.4878 113.6889) (width 0.2) (layer F.Cu) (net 12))
 (via (at 174.1424 113.0554) (size 0.51) (drill 0.3) (layers F.Cu B.Cu) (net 12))
 (segment (start 174.0971 113.6889) (end 174.0971 113.1007) (width 0.2) (layer F.Cu) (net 12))
 (segment (start 174.0971 113.1007) (end 174.1424 113.0554) (width 0.2) (layer F.Cu) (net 12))
 (segment (start 171.5897 107.6833) (end 171.3865 107.4801) (width 0.2) (layer B.Cu) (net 12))
 (segment (start 171.5897 108.3945) (end 171.5897 107.6833) (width 0.2) (layer B.Cu) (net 12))
 (segment (start 174.1424 113.0554) (end 174.1424 110.9472) (width 0.2) (layer B.Cu) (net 12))
 (segment (start 174.1424 110.9472) (end 171.5897 108.3945) (width 0.2) (layer B.Cu) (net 12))
 (via (at 165.5445 106.5911) (size 0.51) (drill 0.3) (layers F.Cu B.Cu) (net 12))
 (segment (start 165.5445 106.5911) (end 165.5445 106.0323) (width 0.2) (layer B.Cu) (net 12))
 (segment (start 166.0144 105.5624) (end 166.8272 105.5624) (width 0.2) (layer B.Cu) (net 12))
 (segment (start 165.5445 106.0323) (end 166.0144 105.5624) (width 0.2) (layer B.Cu) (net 12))
 (segment (start 166.428 113.3968) (end 166.0256 113.3968) (width 0.2) (layer F.Cu) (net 12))
 (segment (start 166.0256 113.3968) (end 165.227 112.5982) (width 0.2) (layer F.Cu) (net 12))
 (segment (start 165.227 106.9086) (end 165.5445 106.5911) (width 0.2) (layer F.Cu) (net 12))
 (segment (start 165.227 112.5982) (end 165.227 106.9086) (width 0.2) (layer F.Cu) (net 12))
 (segment (start 167.774 113.8428) (end 167.774 113.8428) (width 0.2) (layer F.Cu) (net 13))
 (segment (start 168.5313 113.8428) (end 168.3512 113.8428) (width 0.2) (layer F.Cu) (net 13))
 (segment (start 167.774 113.8428) (end 167.328 113.3968) (width 0.2) (layer F.Cu) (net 13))
 (via (at 169.5196 104.4829) (size 0.51) (drill 0.3) (layers F.Cu B.Cu) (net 13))
 (segment (start 166.1088 106.3045) (end 166.6733 106.3045) (width 0.2) (layer F.Cu) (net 13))
 (segment (start 165.9128 106.1085) (end 166.1088 106.3045) (width 0.2) (layer F.Cu) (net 13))
 (segment (start 165.9128 104.7623) (end 165.9128 106.1085) (width 0.2) (layer F.Cu) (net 13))
 (segment (start 169.5196 104.4829) (end 166.1922 104.4829) (width 0.2) (layer F.Cu) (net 13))
 (segment (start 166.1922 104.4829) (end 165.9128 104.7623) (width 0.2) (layer F.Cu) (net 13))
 (segment (start 168.3512 113.8428) (end 167.774 113.8428) (width 0.2) (layer F.Cu) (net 13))
 (via (at 168.3512 113.8428) (size 0.51) (drill 0.3) (layers F.Cu B.Cu) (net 13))
 (segment (start 168.3512 113.8428) (end 168.3512 114.9731) (width 0.2) (layer B.Cu) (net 13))
 (segment (start 170.6499 104.4829) (end 171.0563 104.8893) (width 0.2) (layer B.Cu) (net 13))
 (segment (start 169.5196 104.4829) (end 170.6499 104.4829) (width 0.2) (layer B.Cu) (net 13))
 (segment (start 169.0497 115.6716) (end 168.3512 114.9731) (width 0.2) (layer B.Cu) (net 13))
 (via (at 174.2059 115.5065) (size 0.51) (drill 0.3) (layers F.Cu B.Cu) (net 13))
 (segment (start 174.0971 115.0889) (end 174.0971 115.3977) (width 0.2) (layer F.Cu) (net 13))
 (segment (start 174.0971 115.3977) (end 174.2059 115.5065) (width 0.2) (layer F.Cu) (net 13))
 (segment (start 174.0408 115.6716) (end 169.0497 115.6716) (width 0.2) (layer B.Cu) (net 13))
 (segment (start 174.2059 115.5065) (end 174.0408 115.6716) (width 0.2) (layer B.Cu) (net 13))
 (segment (start 166.6733 106.364) (end 166.6733 106.3045) (width 0.2) (layer F.Cu) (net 13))
 (segment (start 166.1088 106.848202) (end 166.1088 106.3045) (width 0.2) (layer F.Cu) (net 13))
 (segment (start 167.328 113.3968) (end 167.328 113.0609) (width 0.2) (layer F.Cu) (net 13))
 (segment (start 166.9288 112.6617) (end 165.8874 112.6617) (width 0.2) (layer F.Cu) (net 13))
 (segment (start 167.328 113.0609) (end 166.9288 112.6617) (width 0.2) (layer F.Cu) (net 13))
 (segment (start 165.8874 112.6617) (end 165.6334 112.4077) (width 0.2) (layer F.Cu) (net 13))
 (segment (start 165.6334 112.4077) (end 165.6334 107.323602) (width 0.2) (layer F.Cu) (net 13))
 (segment (start 165.6334 107.323602) (end 166.1088 106.848202) (width 0.2) (layer F.Cu) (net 13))
 (via (at 168.3654 108.2802) (size 0.51) (drill 0.3) (layers F.Cu B.Cu) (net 10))
 (segment (start 168.275 106.9825) (end 168.275 108.1898) (width 0.2) (layer B.Cu) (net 10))
 (segment (start 168.275 108.1898) (end 168.3654 108.2802) (width 0.2) (layer B.Cu) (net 10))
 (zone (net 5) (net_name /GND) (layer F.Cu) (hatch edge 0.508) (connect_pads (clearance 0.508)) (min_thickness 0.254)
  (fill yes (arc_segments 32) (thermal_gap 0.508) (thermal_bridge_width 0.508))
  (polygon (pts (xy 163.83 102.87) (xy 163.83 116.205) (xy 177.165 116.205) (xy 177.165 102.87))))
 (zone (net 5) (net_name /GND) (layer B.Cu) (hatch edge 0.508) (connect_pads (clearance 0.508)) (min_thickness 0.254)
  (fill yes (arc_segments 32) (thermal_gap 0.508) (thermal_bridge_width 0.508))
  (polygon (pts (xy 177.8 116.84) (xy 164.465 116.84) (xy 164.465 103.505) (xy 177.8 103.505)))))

